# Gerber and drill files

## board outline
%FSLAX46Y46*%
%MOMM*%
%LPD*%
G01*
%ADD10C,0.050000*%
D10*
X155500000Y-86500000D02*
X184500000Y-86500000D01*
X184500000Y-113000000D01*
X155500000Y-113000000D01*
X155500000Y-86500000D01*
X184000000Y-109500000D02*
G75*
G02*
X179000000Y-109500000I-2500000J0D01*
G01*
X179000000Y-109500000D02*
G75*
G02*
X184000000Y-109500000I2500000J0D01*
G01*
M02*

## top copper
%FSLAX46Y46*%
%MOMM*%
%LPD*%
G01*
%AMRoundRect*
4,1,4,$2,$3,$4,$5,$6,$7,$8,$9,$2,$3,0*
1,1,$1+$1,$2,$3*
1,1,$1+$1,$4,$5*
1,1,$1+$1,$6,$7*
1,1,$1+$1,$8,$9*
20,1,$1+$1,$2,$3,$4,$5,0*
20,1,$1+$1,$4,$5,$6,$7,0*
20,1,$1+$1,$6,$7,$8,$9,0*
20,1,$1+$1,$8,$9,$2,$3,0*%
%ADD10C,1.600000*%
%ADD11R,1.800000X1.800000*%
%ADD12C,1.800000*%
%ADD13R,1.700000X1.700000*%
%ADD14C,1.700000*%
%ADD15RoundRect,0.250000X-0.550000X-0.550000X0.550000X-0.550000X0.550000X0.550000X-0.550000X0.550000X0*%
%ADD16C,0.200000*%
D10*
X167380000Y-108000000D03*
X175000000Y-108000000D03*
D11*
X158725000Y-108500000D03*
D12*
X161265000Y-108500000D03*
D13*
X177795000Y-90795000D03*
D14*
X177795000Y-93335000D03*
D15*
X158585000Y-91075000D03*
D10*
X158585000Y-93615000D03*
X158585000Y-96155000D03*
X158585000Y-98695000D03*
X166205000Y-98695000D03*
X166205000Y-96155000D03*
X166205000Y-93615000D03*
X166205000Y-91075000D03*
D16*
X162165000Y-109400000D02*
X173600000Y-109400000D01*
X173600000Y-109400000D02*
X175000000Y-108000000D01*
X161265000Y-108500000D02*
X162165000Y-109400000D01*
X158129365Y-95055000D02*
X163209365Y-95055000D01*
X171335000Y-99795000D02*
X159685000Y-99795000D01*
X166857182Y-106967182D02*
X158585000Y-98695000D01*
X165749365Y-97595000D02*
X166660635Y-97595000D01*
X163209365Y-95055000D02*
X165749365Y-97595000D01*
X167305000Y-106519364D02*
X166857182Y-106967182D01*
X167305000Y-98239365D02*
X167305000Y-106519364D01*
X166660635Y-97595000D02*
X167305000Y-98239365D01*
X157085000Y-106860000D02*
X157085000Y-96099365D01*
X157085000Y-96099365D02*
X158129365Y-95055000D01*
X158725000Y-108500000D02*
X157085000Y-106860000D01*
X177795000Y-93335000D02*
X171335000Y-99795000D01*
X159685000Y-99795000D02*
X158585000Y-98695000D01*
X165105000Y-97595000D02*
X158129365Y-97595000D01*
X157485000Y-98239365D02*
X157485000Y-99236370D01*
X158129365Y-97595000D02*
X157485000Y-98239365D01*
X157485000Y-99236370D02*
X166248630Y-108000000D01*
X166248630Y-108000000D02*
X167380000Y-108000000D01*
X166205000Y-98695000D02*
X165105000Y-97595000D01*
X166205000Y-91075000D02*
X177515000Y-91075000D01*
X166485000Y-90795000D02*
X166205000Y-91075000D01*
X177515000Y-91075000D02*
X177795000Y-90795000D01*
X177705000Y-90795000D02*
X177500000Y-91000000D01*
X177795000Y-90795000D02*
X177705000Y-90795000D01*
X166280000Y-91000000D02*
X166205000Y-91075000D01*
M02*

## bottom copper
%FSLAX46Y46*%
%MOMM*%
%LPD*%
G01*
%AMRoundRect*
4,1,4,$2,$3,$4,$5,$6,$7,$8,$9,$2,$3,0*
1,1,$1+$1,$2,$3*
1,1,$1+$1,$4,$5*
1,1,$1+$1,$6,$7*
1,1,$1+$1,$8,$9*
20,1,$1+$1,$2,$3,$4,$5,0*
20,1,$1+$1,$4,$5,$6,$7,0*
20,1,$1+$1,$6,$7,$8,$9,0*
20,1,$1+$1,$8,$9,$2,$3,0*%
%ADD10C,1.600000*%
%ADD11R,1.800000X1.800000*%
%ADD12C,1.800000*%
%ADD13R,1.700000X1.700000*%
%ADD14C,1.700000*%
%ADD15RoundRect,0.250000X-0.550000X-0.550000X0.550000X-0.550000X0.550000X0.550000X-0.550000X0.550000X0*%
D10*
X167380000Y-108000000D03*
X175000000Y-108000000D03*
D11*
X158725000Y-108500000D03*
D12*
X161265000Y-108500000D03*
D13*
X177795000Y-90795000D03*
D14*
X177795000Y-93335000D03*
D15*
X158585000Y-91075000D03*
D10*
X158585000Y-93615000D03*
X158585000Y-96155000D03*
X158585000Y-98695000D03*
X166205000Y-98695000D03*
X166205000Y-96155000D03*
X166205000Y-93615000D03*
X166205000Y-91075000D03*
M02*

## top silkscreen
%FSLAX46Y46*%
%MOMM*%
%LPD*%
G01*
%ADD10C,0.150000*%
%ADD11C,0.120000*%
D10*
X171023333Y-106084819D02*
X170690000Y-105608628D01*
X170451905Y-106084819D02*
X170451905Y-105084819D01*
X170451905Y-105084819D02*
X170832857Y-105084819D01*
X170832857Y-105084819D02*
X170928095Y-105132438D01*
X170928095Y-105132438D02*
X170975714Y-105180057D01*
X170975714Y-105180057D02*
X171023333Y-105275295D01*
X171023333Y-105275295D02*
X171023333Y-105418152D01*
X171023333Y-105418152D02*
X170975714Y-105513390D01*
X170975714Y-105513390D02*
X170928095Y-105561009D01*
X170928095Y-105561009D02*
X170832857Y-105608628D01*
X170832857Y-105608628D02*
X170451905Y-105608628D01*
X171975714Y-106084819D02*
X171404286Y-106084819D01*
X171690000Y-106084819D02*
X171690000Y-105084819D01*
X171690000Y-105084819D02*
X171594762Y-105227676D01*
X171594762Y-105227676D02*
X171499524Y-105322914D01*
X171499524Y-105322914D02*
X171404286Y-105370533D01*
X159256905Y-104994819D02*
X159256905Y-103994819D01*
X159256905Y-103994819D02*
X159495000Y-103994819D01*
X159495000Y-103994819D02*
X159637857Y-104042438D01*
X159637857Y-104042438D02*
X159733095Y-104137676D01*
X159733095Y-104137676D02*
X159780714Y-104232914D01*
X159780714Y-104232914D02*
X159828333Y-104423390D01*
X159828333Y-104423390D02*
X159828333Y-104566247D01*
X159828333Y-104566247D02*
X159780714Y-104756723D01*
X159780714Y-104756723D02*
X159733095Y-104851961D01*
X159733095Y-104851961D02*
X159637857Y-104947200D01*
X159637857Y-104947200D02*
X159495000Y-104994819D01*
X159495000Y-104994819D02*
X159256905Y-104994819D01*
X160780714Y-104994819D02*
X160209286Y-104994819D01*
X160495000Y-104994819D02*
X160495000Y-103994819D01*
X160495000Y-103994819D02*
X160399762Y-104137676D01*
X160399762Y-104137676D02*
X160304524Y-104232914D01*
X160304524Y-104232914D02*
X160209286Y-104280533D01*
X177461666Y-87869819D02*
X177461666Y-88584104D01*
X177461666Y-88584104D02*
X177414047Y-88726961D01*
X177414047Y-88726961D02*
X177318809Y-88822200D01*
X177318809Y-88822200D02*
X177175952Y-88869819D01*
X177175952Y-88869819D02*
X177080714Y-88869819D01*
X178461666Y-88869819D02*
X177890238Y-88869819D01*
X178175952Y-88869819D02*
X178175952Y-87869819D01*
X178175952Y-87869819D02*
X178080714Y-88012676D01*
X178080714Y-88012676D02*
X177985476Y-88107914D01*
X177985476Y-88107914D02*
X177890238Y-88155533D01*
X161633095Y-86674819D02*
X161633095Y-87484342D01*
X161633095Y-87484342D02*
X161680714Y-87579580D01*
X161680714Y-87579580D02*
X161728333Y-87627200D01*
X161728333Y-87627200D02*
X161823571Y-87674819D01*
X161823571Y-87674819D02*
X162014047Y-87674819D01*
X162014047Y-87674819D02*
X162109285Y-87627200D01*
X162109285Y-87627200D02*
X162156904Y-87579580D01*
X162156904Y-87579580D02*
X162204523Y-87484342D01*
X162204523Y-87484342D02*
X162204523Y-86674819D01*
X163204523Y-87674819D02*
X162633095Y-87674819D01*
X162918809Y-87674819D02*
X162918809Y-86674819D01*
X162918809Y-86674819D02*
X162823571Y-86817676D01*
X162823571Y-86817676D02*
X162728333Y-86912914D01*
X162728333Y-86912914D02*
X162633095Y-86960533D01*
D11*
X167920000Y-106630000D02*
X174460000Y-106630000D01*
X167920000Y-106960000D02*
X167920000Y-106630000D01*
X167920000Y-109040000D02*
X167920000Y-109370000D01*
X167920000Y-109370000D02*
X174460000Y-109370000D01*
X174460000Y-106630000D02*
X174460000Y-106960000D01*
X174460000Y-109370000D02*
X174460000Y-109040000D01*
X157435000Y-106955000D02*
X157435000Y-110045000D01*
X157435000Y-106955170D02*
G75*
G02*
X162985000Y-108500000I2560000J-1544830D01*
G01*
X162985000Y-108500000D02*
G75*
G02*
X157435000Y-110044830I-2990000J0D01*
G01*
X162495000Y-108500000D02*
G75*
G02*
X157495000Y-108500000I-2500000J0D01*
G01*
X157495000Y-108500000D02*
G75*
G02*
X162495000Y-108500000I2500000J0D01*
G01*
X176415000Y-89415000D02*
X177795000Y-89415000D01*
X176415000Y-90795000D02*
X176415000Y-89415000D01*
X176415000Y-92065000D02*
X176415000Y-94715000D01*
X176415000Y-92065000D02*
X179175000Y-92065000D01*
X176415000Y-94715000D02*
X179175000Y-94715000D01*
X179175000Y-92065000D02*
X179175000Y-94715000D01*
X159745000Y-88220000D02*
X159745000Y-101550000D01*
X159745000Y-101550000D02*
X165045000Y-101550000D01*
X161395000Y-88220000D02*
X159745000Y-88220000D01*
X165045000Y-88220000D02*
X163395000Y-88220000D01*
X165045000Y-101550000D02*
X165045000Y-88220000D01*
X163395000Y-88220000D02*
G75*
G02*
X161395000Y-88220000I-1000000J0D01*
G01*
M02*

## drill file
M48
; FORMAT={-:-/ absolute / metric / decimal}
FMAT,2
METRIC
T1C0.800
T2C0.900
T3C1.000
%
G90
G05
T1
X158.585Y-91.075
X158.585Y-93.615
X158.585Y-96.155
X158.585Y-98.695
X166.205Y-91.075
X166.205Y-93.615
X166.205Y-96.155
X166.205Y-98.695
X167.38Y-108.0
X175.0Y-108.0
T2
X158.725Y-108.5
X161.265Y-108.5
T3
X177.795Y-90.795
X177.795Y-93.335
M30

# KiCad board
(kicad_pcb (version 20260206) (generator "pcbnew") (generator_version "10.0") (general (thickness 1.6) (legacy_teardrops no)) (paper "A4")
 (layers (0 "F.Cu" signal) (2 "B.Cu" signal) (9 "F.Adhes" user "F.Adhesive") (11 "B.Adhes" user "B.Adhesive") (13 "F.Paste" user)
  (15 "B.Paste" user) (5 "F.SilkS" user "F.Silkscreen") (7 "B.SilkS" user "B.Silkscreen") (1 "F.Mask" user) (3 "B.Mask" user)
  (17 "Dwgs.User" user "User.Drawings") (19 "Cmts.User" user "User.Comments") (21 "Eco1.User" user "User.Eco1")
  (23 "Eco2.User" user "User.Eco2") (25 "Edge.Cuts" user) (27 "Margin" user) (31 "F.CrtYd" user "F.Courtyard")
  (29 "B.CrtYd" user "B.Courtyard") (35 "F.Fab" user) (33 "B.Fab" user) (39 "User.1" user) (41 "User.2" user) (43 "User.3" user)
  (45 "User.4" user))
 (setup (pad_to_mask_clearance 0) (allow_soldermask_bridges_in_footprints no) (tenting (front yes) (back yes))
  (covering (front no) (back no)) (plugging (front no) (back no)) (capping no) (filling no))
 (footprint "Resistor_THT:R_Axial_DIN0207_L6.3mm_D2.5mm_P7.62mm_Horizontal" (layer "F.Cu") (at 167.38 108)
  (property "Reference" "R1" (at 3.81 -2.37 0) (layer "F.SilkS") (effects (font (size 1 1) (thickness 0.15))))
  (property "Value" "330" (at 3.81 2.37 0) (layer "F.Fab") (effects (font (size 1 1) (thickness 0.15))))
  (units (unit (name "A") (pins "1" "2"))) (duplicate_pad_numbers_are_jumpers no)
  (fp_line (start 0.54 -1.37) (end 7.08 -1.37) (stroke (width 0.12) (type solid)) (layer "F.SilkS"))
  (fp_line (start 0.54 -1.04) (end 0.54 -1.37) (stroke (width 0.12) (type solid)) (layer "F.SilkS"))
  (fp_line (start 0.54 1.04) (end 0.54 1.37) (stroke (width 0.12) (type solid)) (layer "F.SilkS"))
  (fp_line (start 0.54 1.37) (end 7.08 1.37) (stroke (width 0.12) (type solid)) (layer "F.SilkS"))
  (fp_line (start 7.08 -1.37) (end 7.08 -1.04) (stroke (width 0.12) (type solid)) (layer "F.SilkS"))
  (fp_line (start 7.08 1.37) (end 7.08 1.04) (stroke (width 0.12) (type solid)) (layer "F.SilkS"))
  (pad "1" thru_hole circle (at 0 0) (size 1.6 1.6) (drill 0.8) (layers "*.Cu" "*.Mask") (remove_unused_layers no)
   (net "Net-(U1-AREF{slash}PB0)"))
  (pad "2" thru_hole circle (at 7.62 0) (size 1.6 1.6) (drill 0.8) (layers "*.Cu" "*.Mask") (remove_unused_layers no) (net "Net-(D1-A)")))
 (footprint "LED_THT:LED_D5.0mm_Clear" (layer "F.Cu") (at 158.725 108.5)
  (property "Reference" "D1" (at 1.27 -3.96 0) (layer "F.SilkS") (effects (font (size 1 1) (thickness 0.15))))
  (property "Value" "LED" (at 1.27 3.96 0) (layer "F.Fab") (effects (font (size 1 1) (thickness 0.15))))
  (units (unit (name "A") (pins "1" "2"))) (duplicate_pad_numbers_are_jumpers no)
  (fp_line (start -1.29 -1.545) (end -1.29 1.545) (stroke (width 0.12) (type solid)) (layer "F.SilkS"))
  (fp_arc (start -1.29 -1.54483) (mid 2.071779 -2.880495) (end 4.26 0) (stroke (width 0.12) (type solid)) (layer "F.SilkS"))
  (fp_arc (start 4.26 0) (mid 2.071779 2.880495) (end -1.29 1.54483) (stroke (width 0.12) (type solid)) (layer "F.SilkS"))
  (fp_circle (center 1.27 0) (end 3.77 0) (stroke (width 0.12) (type solid)) (fill no) (layer "F.SilkS"))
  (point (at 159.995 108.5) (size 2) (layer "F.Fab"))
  (pad "1" thru_hole rect (at 0 0) (size 1.8 1.8) (drill 0.9) (layers "*.Cu" "*.Mask") (remove_unused_layers no) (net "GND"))
  (pad "2" thru_hole circle (at 2.54 0) (size 1.8 1.8) (drill 0.9) (layers "*.Cu" "*.Mask") (remove_unused_layers no) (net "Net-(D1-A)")))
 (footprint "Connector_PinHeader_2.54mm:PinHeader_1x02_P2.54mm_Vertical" (layer "F.Cu") (at 177.795 90.795)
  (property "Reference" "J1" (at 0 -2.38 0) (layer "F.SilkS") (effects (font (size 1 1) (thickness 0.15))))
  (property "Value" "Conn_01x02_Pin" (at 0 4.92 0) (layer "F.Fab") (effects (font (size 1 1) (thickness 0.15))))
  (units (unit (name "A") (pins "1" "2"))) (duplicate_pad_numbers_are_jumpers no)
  (fp_line (start -1.38 -1.38) (end 0 -1.38) (stroke (width 0.12) (type solid)) (layer "F.SilkS"))
  (fp_line (start -1.38 0) (end -1.38 -1.38) (stroke (width 0.12) (type solid)) (layer "F.SilkS"))
  (fp_line (start -1.38 1.27) (end -1.38 3.92) (stroke (width 0.12) (type solid)) (layer "F.SilkS"))
  (fp_line (start -1.38 1.27) (end 1.38 1.27) (stroke (width 0.12) (type solid)) (layer "F.SilkS"))
  (fp_line (start -1.38 3.92) (end 1.38 3.92) (stroke (width 0.12) (type solid)) (layer "F.SilkS"))
  (fp_line (start 1.38 1.27) (end 1.38 3.92) (stroke (width 0.12) (type solid)) (layer "F.SilkS"))
  (pad "1" thru_hole rect (at 0 0) (size 1.7 1.7) (drill 1) (layers "*.Cu" "*.Mask") (remove_unused_layers no) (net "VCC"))
  (pad "2" thru_hole circle (at 0 2.54) (size 1.7 1.7) (drill 1) (layers "*.Cu" "*.Mask") (remove_unused_layers no) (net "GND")))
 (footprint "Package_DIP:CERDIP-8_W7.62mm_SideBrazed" (layer "F.Cu") (at 158.585 91.075)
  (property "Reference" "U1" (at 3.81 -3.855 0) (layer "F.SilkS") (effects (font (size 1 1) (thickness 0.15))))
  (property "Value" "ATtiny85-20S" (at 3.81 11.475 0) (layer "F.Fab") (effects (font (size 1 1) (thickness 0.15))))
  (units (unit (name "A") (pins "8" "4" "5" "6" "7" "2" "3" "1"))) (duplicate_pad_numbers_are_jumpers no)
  (fp_line (start 1.16 -2.855) (end 1.16 10.475) (stroke (width 0.12) (type solid)) (layer "F.SilkS"))
  (fp_line (start 1.16 10.475) (end 6.46 10.475) (stroke (width 0.12) (type solid)) (layer "F.SilkS"))
  (fp_line (start 2.81 -2.855) (end 1.16 -2.855) (stroke (width 0.12) (type solid)) (layer "F.SilkS"))
  (fp_line (start 6.46 -2.855) (end 4.81 -2.855) (stroke (width 0.12) (type solid)) (layer "F.SilkS"))
  (fp_line (start 6.46 10.475) (end 6.46 -2.855) (stroke (width 0.12) (type solid)) (layer "F.SilkS"))
  (fp_arc (start 4.81 -2.855) (mid 3.81 -1.855) (end 2.81 -2.855) (stroke (width 0.12) (type solid)) (layer "F.SilkS"))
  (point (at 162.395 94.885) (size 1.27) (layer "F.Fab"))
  (pad "1" thru_hole roundrect (at 0 0) (size 1.6 1.6) (drill 0.8) (layers "*.Cu" "*.Mask") (remove_unused_layers no)
   (roundrect_rratio 0.15625) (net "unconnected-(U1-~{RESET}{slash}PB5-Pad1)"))
  (pad "2" thru_hole circle (at 0 2.54) (size 1.6 1.6) (drill 0.8) (layers "*.Cu" "*.Mask") (remove_unused_layers no)
   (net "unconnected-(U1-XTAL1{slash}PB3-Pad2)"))
  (pad "3" thru_hole circle (at 0 5.08) (size 1.6 1.6) (drill 0.8) (layers "*.Cu" "*.Mask") (remove_unused_layers no)
   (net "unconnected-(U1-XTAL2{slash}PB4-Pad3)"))
  (pad "4" thru_hole circle (at 0 7.62) (size 1.6 1.6) (drill 0.8) (layers "*.Cu" "*.Mask") (remove_unused_layers no) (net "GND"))
  (pad "5" thru_hole circle (at 7.62 7.62) (size 1.6 1.6) (drill 0.8) (layers "*.Cu" "*.Mask") (remove_unused_layers no)
   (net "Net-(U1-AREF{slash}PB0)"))
  (pad "6" thru_hole circle (at 7.62 5.08) (size 1.6 1.6) (drill 0.8) (layers "*.Cu" "*.Mask") (remove_unused_layers no)
   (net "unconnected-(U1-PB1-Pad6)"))
  (pad "7" thru_hole circle (at 7.62 2.54) (size 1.6 1.6) (drill 0.8) (layers "*.Cu" "*.Mask") (remove_unused_layers no)
   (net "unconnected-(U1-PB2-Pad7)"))
  (pad "8" thru_hole circle (at 7.62 0) (size 1.6 1.6) (drill 0.8) (layers "*.Cu" "*.Mask") (remove_unused_layers no) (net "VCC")))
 (gr_rect (start 155.5 86.5) (end 184.5 113) (stroke (width 0.05) (type default)) (fill no) (layer "Edge.Cuts"))
 (gr_circle (center 181.5 109.5) (end 180 107.5) (stroke (width 0.05) (type default)) (fill no) (layer "Edge.Cuts"))
 (segment (start 162.165 109.4) (end 173.6 109.4) (width 0.2) (layer "F.Cu") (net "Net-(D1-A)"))
 (segment (start 173.6 109.4) (end 175 108) (width 0.2) (layer "F.Cu") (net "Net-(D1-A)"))
 (segment (start 161.265 108.5) (end 162.165 109.4) (width 0.2) (layer "F.Cu") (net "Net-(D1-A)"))
 (segment (start 158.129365 95.055) (end 163.209365 95.055) (width 0.2) (layer "F.Cu") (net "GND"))
 (segment (start 171.335 99.795) (end 159.685 99.795) (width 0.2) (layer "F.Cu") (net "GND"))
 (segment (start 166.857182 106.967182) (end 158.585 98.695) (width 0.2) (layer "F.Cu") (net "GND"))
 (segment (start 165.749365 97.595) (end 166.660635 97.595) (width 0.2) (layer "F.Cu") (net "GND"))
 (segment (start 163.209365 95.055) (end 165.749365 97.595) (width 0.2) (layer "F.Cu") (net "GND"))
 (segment (start 167.305 106.519364) (end 166.857182 106.967182) (width 0.2) (layer "F.Cu") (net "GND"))
 (segment (start 167.305 98.239365) (end 167.305 106.519364) (width 0.2) (layer "F.Cu") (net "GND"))
 (segment (start 166.660635 97.595) (end 167.305 98.239365) (width 0.2) (layer "F.Cu") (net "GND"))
 (segment (start 157.085 106.86) (end 157.085 96.099365) (width 0.2) (layer "F.Cu") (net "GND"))
 (segment (start 157.085 96.099365) (end 158.129365 95.055) (width 0.2) (layer "F.Cu") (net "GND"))
 (segment (start 158.725 108.5) (end 157.085 106.86) (width 0.2) (layer "F.Cu") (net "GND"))
 (segment (start 177.795 93.335) (end 171.335 99.795) (width 0.2) (layer "F.Cu") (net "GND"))
 (segment (start 159.685 99.795) (end 158.585 98.695) (width 0.2) (layer "F.Cu") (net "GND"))
 (segment (start 165.105 97.595) (end 158.129365 97.595) (width 0.2) (layer "F.Cu") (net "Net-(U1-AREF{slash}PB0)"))
 (segment (start 157.485 98.239365) (end 157.485 99.23637) (width 0.2) (layer "F.Cu") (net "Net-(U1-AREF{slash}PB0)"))
 (segment (start 158.129365 97.595) (end 157.485 98.239365) (width 0.2) (layer "F.Cu") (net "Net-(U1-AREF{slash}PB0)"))
 (segment (start 157.485 99.23637) (end 166.24863 108) (width 0.2) (layer "F.Cu") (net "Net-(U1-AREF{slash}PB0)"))
 (segment (start 166.24863 108) (end 167.38 108) (width 0.2) (layer "F.Cu") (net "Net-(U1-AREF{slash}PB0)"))
 (segment (start 166.205 98.695) (end 165.105 97.595) (width 0.2) (layer "F.Cu") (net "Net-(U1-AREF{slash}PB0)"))
 (segment (start 166.205 91.075) (end 177.515 91.075) (width 0.2) (layer "F.Cu") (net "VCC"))
 (segment (start 166.485 90.795) (end 166.205 91.075) (width 0.2) (layer "F.Cu") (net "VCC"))
 (segment (start 177.515 91.075) (end 177.795 90.795) (width 0.2) (layer "F.Cu") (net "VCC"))
 (segment (start 177.705 90.795) (end 177.5 91) (width 0.2) (layer "F.Cu") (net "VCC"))
 (segment (start 177.795 90.795) (end 177.705 90.795) (width 0.2) (layer "F.Cu") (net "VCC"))
 (segment (start 166.28 91) (end 166.205 91.075) (width 0.2) (layer "F.Cu") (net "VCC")))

